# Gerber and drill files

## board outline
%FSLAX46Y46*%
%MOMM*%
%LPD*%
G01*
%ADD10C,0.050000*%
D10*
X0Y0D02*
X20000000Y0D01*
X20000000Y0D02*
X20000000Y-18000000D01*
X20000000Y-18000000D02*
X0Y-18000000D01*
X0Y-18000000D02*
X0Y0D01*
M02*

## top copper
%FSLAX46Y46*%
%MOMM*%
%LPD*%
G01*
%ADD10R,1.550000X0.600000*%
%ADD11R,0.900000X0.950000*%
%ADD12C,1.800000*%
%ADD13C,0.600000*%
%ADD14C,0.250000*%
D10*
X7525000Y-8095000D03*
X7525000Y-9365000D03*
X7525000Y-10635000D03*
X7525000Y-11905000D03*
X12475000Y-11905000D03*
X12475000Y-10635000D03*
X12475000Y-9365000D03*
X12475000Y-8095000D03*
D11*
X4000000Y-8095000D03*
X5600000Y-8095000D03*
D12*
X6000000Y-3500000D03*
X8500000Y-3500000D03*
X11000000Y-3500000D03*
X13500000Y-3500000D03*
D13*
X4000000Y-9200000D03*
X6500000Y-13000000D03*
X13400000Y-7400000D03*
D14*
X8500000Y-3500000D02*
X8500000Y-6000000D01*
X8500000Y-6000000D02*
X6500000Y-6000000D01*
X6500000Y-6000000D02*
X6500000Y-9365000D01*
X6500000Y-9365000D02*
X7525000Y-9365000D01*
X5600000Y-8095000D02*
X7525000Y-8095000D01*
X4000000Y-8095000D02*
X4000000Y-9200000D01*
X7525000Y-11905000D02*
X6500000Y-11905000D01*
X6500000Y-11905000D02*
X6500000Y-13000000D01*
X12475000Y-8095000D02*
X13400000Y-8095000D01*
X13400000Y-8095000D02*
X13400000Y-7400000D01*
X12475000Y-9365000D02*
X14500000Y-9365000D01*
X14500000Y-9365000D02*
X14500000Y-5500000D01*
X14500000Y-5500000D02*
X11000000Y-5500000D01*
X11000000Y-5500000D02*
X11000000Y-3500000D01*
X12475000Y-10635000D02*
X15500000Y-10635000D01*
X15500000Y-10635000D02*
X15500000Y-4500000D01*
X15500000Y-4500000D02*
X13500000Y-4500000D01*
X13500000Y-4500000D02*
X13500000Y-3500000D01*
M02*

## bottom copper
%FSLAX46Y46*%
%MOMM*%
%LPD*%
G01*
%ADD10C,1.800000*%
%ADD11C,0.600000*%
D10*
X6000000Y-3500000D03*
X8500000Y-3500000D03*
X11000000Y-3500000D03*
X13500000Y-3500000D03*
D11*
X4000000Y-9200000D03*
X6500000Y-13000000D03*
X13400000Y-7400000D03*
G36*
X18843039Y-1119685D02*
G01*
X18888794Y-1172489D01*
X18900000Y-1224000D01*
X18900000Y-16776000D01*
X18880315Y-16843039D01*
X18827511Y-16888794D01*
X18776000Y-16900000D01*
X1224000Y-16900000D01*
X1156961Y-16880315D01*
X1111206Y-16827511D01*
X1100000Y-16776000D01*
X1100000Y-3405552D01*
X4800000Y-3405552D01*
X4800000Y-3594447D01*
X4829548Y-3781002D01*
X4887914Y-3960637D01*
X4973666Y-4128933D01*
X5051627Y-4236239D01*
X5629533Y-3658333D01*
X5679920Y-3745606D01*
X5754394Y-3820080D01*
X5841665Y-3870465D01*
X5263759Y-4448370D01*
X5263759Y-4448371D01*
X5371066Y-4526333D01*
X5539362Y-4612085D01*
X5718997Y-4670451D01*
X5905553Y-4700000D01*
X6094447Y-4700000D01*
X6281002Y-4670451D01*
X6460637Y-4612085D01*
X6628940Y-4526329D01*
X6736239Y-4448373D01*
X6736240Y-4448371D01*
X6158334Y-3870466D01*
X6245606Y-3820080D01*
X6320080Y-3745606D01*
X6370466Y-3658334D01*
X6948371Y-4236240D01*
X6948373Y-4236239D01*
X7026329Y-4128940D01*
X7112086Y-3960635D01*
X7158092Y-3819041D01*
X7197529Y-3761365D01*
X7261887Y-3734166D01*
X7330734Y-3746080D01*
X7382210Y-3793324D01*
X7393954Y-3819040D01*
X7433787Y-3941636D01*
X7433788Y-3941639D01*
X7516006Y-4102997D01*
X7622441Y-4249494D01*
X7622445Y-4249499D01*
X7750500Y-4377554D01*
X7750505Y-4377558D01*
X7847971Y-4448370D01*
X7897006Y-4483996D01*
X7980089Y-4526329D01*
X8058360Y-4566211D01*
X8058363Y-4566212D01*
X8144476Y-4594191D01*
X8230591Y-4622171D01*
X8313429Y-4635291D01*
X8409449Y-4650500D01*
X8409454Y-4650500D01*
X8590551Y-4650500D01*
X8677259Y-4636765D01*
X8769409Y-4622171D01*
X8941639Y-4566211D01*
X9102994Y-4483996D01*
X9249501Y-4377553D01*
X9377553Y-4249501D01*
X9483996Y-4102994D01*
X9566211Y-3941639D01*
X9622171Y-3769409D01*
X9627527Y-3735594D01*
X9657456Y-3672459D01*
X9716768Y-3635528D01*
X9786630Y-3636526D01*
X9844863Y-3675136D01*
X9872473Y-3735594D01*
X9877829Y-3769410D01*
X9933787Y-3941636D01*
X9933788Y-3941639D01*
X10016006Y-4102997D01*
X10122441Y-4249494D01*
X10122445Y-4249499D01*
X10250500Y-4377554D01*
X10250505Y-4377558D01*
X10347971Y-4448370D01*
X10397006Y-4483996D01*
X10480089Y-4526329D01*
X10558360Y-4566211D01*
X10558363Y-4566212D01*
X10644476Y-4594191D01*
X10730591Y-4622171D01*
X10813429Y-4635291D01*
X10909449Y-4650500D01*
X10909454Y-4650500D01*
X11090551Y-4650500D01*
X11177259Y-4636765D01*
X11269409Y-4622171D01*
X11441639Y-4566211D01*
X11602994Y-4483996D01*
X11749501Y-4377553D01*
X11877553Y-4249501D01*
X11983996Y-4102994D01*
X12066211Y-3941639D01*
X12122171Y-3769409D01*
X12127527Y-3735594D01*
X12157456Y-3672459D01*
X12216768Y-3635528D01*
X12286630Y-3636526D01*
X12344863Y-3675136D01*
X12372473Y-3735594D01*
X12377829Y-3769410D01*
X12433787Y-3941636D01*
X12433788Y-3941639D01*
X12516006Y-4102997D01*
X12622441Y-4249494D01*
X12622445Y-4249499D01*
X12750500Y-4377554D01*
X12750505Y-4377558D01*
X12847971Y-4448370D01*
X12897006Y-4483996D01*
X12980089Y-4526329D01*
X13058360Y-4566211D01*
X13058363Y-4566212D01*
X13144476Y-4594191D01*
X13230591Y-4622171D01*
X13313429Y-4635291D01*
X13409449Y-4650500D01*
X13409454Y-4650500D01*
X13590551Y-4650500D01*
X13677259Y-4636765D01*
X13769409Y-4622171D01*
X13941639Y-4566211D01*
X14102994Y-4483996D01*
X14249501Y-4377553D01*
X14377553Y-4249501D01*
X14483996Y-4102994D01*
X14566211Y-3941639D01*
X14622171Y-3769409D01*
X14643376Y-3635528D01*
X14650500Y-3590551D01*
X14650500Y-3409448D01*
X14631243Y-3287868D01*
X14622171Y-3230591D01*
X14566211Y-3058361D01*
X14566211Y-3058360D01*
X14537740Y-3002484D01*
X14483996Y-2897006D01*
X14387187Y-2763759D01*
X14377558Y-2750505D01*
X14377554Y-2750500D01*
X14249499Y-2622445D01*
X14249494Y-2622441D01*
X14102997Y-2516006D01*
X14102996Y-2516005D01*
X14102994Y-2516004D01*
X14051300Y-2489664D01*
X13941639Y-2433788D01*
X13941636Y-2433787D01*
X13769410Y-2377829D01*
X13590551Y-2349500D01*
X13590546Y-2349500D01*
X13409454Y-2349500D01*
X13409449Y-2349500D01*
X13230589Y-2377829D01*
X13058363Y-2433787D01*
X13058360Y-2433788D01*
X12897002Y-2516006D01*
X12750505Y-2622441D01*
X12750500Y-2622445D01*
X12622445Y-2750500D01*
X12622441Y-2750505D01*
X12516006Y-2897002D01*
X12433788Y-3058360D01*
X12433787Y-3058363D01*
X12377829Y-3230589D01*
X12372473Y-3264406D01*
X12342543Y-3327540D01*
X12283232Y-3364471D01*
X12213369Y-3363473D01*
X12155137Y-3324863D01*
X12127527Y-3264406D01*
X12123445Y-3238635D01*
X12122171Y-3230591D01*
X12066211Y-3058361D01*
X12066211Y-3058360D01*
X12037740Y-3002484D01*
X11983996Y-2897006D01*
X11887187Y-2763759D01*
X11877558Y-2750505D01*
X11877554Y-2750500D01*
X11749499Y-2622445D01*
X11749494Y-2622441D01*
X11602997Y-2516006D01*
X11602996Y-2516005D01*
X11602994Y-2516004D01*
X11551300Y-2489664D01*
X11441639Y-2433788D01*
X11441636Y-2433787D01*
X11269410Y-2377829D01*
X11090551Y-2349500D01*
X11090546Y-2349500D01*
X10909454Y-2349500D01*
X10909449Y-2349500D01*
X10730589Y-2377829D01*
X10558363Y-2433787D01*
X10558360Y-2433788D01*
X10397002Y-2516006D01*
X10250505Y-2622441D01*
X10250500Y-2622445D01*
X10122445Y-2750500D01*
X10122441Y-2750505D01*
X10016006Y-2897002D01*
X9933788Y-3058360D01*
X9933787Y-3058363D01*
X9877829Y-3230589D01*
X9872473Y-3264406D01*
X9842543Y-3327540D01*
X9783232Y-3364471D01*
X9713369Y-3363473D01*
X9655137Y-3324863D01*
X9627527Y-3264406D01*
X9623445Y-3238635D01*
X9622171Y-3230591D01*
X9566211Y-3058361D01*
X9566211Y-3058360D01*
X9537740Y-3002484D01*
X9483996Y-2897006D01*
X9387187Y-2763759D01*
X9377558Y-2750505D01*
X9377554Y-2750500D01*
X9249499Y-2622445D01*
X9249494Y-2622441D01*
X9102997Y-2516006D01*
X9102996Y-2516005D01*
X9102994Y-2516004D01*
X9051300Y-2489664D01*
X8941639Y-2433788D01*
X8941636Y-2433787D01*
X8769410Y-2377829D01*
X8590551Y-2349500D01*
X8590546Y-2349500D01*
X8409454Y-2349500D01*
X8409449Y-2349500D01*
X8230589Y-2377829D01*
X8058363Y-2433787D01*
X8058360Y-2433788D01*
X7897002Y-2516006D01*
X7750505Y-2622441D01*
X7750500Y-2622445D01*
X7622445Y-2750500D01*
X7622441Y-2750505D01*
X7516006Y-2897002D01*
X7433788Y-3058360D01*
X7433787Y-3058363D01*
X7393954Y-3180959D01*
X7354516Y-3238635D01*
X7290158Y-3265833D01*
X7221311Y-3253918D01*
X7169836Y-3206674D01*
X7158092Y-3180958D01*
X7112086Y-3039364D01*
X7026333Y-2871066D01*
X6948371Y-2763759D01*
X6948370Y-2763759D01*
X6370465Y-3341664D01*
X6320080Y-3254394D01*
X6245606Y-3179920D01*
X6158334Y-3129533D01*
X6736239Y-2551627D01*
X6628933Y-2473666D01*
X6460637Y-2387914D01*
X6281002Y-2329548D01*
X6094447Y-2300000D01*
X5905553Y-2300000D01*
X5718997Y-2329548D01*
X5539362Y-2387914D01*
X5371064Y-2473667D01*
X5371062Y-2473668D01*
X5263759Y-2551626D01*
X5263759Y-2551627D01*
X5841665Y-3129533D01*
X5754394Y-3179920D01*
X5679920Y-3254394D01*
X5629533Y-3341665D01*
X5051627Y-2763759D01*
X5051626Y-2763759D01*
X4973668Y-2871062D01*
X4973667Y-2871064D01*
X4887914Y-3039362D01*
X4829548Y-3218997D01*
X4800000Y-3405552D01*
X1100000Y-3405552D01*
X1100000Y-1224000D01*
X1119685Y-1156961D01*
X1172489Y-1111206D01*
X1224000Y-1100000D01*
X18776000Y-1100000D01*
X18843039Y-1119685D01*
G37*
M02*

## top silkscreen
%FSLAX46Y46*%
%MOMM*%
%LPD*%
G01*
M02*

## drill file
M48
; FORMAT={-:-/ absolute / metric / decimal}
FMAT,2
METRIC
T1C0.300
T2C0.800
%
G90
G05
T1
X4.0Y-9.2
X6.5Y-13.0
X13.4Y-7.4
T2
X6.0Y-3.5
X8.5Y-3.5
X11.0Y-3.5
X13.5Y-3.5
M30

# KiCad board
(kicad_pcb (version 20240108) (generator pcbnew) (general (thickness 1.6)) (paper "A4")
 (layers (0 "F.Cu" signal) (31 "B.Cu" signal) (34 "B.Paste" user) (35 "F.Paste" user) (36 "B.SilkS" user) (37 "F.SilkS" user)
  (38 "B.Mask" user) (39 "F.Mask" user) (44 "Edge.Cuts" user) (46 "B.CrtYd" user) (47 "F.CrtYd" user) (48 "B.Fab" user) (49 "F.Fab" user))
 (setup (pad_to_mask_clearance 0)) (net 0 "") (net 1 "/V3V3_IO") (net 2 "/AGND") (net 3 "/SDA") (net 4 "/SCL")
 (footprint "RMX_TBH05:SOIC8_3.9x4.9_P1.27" (layer "F.Cu") (at 10 10)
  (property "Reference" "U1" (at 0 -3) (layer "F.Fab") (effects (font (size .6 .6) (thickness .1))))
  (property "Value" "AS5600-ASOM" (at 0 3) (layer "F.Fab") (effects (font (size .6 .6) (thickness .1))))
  (pad "1" smd rect (at -2.475 -1.905) (size 1.55 0.6) (layers "F.Cu" "F.Paste" "F.Mask") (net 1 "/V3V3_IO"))
  (pad "2" smd rect (at -2.475 -0.635) (size 1.55 0.6) (layers "F.Cu" "F.Paste" "F.Mask") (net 1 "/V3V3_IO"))
  (pad "3" smd rect (at -2.475 0.635) (size 1.55 0.6) (layers "F.Cu" "F.Paste" "F.Mask"))
  (pad "4" smd rect (at -2.475 1.905) (size 1.55 0.6) (layers "F.Cu" "F.Paste" "F.Mask") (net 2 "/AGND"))
  (pad "5" smd rect (at 2.475 1.905) (size 1.55 0.6) (layers "F.Cu" "F.Paste" "F.Mask"))
  (pad "6" smd rect (at 2.475 0.635) (size 1.55 0.6) (layers "F.Cu" "F.Paste" "F.Mask") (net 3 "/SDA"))
  (pad "7" smd rect (at 2.475 -0.635) (size 1.55 0.6) (layers "F.Cu" "F.Paste" "F.Mask") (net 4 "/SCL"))
  (pad "8" smd rect (at 2.475 -1.905) (size 1.55 0.6) (layers "F.Cu" "F.Paste" "F.Mask") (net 2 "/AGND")))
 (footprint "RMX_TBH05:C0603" (layer "F.Cu") (at 4.8 8.095)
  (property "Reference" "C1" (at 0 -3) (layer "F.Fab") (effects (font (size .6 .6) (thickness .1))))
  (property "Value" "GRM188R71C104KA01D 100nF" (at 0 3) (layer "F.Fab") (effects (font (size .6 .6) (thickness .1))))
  (pad "1" smd rect (at -0.8 0) (size 0.9 0.95) (layers "F.Cu" "F.Paste" "F.Mask") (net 2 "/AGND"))
  (pad "2" smd rect (at 0.8 0) (size 0.9 0.95) (layers "F.Cu" "F.Paste" "F.Mask") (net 1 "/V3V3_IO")))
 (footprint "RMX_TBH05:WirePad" (layer "F.Cu") (at 6 3.5)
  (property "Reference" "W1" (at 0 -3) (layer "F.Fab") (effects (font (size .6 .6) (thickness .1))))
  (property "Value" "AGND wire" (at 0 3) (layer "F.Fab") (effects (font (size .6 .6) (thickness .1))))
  (pad "1" thru_hole circle (at 0 0) (size 1.8 1.8) (drill 0.8) (layers "*.Cu" "*.Mask") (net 2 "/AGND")))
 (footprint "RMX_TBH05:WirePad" (layer "F.Cu") (at 8.5 3.5)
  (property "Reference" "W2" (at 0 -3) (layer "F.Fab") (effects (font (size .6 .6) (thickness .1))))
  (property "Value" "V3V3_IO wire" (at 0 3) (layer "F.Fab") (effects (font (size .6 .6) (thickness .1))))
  (pad "1" thru_hole circle (at 0 0) (size 1.8 1.8) (drill 0.8) (layers "*.Cu" "*.Mask") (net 1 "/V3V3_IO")))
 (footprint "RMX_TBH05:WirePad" (layer "F.Cu") (at 11 3.5)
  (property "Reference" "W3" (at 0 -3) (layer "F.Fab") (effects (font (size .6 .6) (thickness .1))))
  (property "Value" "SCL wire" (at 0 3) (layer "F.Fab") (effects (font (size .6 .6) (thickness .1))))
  (pad "1" thru_hole circle (at 0 0) (size 1.8 1.8) (drill 0.8) (layers "*.Cu" "*.Mask") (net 4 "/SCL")))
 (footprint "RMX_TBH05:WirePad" (layer "F.Cu") (at 13.5 3.5)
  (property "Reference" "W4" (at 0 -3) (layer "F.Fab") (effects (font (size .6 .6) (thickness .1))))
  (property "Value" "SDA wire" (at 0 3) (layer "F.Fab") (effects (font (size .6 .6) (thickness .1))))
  (pad "1" thru_hole circle (at 0 0) (size 1.8 1.8) (drill 0.8) (layers "*.Cu" "*.Mask") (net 3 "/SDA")))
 (segment (start 8.5 3.5) (end 8.5 6) (width 0.25) (layer "F.Cu") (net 1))
 (segment (start 8.5 6) (end 6.5 6) (width 0.25) (layer "F.Cu") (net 1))
 (segment (start 6.5 6) (end 6.5 9.365) (width 0.25) (layer "F.Cu") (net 1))
 (segment (start 6.5 9.365) (end 7.525 9.365) (width 0.25) (layer "F.Cu") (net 1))
 (segment (start 5.6 8.095) (end 7.525 8.095) (width 0.25) (layer "F.Cu") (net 1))
 (segment (start 4 8.095) (end 4 9.2) (width 0.25) (layer "F.Cu") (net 2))
 (segment (start 7.525 11.905) (end 6.5 11.905) (width 0.25) (layer "F.Cu") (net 2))
 (segment (start 6.5 11.905) (end 6.5 13) (width 0.25) (layer "F.Cu") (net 2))
 (segment (start 12.475 8.095) (end 13.4 8.095) (width 0.25) (layer "F.Cu") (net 2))
 (segment (start 13.4 8.095) (end 13.4 7.4) (width 0.25) (layer "F.Cu") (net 2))
 (segment (start 12.475 9.365) (end 14.5 9.365) (width 0.25) (layer "F.Cu") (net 4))
 (segment (start 14.5 9.365) (end 14.5 5.5) (width 0.25) (layer "F.Cu") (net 4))
 (segment (start 14.5 5.5) (end 11 5.5) (width 0.25) (layer "F.Cu") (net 4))
 (segment (start 11 5.5) (end 11 3.5) (width 0.25) (layer "F.Cu") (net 4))
 (segment (start 12.475 10.635) (end 15.5 10.635) (width 0.25) (layer "F.Cu") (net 3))
 (segment (start 15.5 10.635) (end 15.5 4.5) (width 0.25) (layer "F.Cu") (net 3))
 (segment (start 15.5 4.5) (end 13.5 4.5) (width 0.25) (layer "F.Cu") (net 3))
 (segment (start 13.5 4.5) (end 13.5 3.5) (width 0.25) (layer "F.Cu") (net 3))
 (via (at 4 9.2) (size .6) (drill .3) (layers "F.Cu" "B.Cu") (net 2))
 (via (at 6.5 13) (size .6) (drill .3) (layers "F.Cu" "B.Cu") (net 2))
 (via (at 13.4 7.4) (size .6) (drill .3) (layers "F.Cu" "B.Cu") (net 2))
 (gr_line (start 0 0) (end 20 0) (stroke (width .05) (type default)) (layer "Edge.Cuts"))
 (gr_line (start 20 0) (end 20 18) (stroke (width .05) (type default)) (layer "Edge.Cuts"))
 (gr_line (start 20 18) (end 0 18) (stroke (width .05) (type default)) (layer "Edge.Cuts"))
 (gr_line (start 0 18) (end 0 0) (stroke (width .05) (type default)) (layer "Edge.Cuts"))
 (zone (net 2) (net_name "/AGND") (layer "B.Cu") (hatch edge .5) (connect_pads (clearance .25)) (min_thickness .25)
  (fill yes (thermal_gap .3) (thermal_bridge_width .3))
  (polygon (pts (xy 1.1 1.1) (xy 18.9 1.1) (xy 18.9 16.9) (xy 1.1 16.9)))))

